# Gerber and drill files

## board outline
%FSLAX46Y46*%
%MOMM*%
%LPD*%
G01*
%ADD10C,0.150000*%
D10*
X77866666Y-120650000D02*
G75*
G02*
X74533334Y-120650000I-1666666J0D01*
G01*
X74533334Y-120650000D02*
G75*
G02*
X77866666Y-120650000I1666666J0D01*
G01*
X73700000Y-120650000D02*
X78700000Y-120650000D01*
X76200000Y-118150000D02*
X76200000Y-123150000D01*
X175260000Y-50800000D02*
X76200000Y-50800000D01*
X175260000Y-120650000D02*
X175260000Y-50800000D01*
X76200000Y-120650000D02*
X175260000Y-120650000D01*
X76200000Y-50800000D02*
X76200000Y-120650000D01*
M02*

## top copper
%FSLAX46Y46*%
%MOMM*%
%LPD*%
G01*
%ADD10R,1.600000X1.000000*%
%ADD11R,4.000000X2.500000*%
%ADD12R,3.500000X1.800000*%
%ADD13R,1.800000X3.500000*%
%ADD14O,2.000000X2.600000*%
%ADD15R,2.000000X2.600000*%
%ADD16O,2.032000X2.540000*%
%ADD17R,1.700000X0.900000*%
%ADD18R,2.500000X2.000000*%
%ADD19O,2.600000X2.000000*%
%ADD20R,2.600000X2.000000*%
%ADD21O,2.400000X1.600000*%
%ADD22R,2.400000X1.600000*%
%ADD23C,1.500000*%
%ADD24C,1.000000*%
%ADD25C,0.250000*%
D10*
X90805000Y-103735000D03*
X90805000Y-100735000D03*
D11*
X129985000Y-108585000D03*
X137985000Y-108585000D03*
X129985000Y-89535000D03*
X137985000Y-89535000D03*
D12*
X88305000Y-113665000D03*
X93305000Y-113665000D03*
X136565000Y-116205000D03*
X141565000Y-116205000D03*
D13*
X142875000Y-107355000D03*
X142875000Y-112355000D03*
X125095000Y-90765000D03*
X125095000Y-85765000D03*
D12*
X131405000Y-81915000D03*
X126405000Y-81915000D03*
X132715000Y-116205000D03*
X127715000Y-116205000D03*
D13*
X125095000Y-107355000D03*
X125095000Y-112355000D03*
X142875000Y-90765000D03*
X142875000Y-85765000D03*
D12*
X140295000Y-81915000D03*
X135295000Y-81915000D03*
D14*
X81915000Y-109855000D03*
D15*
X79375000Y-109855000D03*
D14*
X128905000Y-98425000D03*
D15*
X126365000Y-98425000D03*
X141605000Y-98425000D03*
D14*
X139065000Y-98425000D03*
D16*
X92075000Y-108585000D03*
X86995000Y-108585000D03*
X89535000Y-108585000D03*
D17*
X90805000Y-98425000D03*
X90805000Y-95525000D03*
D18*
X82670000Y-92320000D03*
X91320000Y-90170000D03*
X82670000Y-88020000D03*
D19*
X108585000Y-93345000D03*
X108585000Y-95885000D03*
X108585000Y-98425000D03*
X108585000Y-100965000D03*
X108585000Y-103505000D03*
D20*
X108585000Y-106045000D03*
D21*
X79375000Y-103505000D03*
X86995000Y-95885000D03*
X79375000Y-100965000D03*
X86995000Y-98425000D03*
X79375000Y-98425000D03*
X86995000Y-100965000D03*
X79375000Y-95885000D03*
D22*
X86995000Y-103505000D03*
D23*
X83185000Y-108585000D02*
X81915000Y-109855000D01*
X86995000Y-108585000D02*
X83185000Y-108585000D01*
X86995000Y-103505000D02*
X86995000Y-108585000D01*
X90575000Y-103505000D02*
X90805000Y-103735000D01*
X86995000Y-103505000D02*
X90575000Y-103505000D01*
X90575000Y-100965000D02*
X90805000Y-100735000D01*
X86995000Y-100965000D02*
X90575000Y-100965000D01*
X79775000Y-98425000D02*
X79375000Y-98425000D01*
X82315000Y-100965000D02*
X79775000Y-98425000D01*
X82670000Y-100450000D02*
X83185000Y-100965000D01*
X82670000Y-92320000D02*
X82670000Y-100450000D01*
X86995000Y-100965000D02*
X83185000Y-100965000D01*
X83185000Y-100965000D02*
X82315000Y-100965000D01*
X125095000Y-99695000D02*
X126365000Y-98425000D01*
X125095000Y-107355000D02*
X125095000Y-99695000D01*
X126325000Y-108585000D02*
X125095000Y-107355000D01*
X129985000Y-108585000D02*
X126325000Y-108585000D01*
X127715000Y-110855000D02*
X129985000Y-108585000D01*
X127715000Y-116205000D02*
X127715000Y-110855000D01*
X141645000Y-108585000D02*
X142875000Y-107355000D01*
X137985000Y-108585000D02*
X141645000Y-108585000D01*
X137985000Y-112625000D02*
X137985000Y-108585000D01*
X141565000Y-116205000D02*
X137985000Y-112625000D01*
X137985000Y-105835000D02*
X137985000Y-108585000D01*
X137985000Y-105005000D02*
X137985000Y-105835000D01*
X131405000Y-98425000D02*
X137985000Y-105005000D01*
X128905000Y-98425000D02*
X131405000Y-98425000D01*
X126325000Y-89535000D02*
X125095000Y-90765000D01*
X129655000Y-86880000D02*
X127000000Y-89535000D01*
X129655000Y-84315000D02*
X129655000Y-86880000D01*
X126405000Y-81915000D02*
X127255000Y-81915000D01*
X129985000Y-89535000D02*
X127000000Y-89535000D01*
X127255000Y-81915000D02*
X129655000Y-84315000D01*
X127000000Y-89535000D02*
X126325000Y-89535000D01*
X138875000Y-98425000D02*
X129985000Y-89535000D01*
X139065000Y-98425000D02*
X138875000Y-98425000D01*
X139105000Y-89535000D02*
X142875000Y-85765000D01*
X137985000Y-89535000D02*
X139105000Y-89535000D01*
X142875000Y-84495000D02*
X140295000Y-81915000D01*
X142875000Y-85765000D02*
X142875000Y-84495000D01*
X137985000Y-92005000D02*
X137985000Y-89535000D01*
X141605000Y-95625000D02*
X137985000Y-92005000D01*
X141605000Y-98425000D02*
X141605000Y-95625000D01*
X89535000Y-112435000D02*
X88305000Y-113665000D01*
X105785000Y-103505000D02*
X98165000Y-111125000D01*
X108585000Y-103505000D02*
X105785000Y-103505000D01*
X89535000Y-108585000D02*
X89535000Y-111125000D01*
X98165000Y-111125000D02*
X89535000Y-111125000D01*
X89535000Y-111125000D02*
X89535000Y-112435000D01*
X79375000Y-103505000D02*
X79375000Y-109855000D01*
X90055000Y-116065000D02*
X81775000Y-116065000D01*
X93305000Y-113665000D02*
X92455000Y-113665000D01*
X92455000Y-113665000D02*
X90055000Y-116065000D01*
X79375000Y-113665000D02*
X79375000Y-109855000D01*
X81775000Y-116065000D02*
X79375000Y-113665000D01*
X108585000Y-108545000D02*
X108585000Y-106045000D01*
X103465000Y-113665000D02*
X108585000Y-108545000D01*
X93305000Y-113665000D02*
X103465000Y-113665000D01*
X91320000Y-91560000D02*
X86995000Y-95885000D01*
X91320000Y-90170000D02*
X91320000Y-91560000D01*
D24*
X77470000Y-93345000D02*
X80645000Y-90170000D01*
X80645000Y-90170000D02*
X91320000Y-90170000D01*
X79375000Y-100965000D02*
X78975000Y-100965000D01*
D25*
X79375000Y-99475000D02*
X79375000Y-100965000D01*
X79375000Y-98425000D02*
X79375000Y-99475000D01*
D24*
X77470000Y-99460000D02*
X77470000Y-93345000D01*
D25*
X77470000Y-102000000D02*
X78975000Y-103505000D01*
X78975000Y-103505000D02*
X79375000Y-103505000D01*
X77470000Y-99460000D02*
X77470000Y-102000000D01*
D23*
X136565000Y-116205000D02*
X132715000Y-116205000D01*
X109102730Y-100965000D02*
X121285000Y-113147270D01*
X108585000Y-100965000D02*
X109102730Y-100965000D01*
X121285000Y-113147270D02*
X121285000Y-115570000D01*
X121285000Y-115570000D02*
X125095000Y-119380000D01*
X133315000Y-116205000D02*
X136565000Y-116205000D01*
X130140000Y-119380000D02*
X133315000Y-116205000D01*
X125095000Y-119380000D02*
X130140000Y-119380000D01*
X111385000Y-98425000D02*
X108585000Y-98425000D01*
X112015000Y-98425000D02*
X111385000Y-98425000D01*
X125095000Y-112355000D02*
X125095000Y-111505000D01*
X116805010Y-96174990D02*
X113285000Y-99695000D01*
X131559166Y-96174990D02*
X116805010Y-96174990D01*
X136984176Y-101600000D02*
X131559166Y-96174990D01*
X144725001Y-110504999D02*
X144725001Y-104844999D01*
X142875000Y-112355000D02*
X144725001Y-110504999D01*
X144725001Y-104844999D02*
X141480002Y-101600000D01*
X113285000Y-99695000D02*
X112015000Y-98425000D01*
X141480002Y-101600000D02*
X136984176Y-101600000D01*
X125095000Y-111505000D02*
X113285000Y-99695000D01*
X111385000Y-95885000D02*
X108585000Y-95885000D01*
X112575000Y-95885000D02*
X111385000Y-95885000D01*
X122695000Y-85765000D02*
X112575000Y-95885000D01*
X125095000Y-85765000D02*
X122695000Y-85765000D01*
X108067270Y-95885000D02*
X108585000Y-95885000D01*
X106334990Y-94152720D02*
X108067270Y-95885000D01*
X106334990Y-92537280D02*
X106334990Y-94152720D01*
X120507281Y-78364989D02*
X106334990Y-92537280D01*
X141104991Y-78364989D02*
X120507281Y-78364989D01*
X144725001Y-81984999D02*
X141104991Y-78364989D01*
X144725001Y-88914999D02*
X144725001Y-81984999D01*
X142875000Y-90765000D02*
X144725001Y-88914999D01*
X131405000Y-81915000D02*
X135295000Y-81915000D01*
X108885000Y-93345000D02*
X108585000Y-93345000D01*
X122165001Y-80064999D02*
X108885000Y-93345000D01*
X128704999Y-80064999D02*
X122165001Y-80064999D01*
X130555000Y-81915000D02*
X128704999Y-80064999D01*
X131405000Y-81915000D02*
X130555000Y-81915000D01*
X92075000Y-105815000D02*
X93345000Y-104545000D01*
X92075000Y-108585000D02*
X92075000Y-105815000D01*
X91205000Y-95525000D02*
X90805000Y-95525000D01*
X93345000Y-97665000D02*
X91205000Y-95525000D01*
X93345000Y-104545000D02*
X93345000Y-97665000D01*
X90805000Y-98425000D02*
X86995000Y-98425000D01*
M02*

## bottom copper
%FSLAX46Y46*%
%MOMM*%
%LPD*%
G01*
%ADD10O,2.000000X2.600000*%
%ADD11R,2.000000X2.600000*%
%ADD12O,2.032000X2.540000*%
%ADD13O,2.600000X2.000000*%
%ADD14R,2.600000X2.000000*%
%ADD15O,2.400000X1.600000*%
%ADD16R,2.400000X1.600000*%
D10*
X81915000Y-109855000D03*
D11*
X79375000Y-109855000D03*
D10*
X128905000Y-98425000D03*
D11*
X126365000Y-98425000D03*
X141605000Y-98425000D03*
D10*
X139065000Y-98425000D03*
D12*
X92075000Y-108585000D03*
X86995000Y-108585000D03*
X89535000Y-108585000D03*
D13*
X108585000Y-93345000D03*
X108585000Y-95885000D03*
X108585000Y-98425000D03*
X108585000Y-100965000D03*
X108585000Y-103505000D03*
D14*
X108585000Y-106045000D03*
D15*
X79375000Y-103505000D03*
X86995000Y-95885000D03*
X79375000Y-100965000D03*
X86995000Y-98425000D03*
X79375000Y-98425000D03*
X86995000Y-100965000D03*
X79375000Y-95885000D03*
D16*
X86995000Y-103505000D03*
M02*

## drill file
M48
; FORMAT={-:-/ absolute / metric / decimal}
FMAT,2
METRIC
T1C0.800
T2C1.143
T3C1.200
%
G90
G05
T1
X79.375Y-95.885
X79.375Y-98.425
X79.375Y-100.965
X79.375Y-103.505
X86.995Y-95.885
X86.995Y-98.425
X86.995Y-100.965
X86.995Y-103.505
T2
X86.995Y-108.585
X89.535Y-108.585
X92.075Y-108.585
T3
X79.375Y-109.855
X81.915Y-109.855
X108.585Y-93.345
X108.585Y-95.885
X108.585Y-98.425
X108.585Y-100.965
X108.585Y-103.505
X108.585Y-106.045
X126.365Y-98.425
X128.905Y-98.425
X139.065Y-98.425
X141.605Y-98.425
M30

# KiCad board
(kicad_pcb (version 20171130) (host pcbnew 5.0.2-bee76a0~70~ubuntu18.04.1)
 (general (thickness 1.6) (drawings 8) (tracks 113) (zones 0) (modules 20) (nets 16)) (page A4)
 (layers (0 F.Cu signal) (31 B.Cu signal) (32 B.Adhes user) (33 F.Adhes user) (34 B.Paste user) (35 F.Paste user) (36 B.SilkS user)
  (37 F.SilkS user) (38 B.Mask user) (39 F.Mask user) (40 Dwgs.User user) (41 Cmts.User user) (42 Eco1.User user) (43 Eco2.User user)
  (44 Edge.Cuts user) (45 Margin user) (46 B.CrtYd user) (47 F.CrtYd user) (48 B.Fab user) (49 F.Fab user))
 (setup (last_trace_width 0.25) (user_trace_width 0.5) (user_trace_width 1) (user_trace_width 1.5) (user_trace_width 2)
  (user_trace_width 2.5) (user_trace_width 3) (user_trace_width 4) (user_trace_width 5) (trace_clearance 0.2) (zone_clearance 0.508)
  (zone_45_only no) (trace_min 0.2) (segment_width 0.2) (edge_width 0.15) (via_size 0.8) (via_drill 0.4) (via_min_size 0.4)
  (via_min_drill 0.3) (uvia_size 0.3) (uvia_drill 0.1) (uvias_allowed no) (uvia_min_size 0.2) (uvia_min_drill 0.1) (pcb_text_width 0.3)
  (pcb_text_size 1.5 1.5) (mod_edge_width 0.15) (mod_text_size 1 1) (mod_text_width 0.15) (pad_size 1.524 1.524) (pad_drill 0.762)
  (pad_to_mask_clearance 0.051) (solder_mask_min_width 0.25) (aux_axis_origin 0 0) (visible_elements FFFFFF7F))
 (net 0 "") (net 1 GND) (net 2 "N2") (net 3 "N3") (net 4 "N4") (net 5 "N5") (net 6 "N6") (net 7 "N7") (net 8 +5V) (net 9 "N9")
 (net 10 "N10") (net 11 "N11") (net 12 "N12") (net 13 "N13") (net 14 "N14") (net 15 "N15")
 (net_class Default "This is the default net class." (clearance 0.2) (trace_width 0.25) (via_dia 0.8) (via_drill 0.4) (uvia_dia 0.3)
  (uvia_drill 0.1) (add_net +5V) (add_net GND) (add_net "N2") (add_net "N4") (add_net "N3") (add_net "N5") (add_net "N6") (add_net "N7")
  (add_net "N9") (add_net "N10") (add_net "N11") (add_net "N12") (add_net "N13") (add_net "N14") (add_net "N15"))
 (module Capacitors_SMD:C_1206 (layer F.Cu) (at 90.805 102.235 270)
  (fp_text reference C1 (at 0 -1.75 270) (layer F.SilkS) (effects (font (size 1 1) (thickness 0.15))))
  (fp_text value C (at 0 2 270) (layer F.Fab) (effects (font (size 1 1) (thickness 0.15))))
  (pad 2 smd rect (at 1.5 0 270) (size 1 1.6) (layers F.Cu F.Paste F.Mask) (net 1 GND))
  (pad 1 smd rect (at -1.5 0 270) (size 1 1.6) (layers F.Cu F.Paste F.Mask) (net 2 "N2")))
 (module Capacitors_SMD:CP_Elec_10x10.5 (layer F.Cu) (at 133.985 108.585 180)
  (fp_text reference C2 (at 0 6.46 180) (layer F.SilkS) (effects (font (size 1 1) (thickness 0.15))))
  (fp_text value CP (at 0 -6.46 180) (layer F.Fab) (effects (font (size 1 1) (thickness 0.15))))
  (pad 2 smd rect (at 4 0) (size 4 2.5) (layers F.Cu F.Paste F.Mask) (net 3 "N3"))
  (pad 1 smd rect (at -4 0) (size 4 2.5) (layers F.Cu F.Paste F.Mask) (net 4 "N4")))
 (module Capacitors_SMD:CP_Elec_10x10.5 (layer F.Cu) (at 133.985 89.535)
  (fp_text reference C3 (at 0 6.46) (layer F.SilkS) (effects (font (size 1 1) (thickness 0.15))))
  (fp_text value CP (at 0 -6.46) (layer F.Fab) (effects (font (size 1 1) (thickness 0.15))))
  (pad 1 smd rect (at -4 0 180) (size 4 2.5) (layers F.Cu F.Paste F.Mask) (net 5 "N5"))
  (pad 2 smd rect (at 4 0 180) (size 4 2.5) (layers F.Cu F.Paste F.Mask) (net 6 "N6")))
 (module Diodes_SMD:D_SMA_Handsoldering (layer F.Cu) (at 90.805 113.665 180)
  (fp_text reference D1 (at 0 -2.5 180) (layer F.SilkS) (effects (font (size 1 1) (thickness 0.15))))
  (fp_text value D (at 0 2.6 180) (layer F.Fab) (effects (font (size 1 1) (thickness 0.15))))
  (pad 2 smd rect (at 2.5 0 180) (size 3.5 1.8) (layers F.Cu F.Paste F.Mask) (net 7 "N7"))
  (pad 1 smd rect (at -2.5 0 180) (size 3.5 1.8) (layers F.Cu F.Paste F.Mask) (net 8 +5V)))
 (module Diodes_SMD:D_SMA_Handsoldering (layer F.Cu) (at 139.065 116.205 180)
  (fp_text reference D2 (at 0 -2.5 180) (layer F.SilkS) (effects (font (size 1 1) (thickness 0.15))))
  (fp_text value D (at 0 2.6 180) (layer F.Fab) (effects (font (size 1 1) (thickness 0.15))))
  (pad 2 smd rect (at 2.5 0 180) (size 3.5 1.8) (layers F.Cu F.Paste F.Mask) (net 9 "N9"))
  (pad 1 smd rect (at -2.5 0 180) (size 3.5 1.8) (layers F.Cu F.Paste F.Mask) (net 4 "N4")))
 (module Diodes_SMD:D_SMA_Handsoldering (layer F.Cu) (at 142.875 109.855 270)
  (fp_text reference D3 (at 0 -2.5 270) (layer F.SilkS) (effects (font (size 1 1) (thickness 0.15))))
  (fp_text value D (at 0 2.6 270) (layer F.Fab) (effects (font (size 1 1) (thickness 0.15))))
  (pad 1 smd rect (at -2.5 0 270) (size 3.5 1.8) (layers F.Cu F.Paste F.Mask) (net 4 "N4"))
  (pad 2 smd rect (at 2.5 0 270) (size 3.5 1.8) (layers F.Cu F.Paste F.Mask) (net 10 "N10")))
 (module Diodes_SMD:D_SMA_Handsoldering (layer F.Cu) (at 125.095 88.265 90)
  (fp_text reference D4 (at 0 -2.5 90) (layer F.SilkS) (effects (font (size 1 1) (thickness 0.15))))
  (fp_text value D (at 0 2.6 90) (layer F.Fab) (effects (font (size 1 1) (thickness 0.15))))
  (pad 1 smd rect (at -2.5 0 90) (size 3.5 1.8) (layers F.Cu F.Paste F.Mask) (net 5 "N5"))
  (pad 2 smd rect (at 2.5 0 90) (size 3.5 1.8) (layers F.Cu F.Paste F.Mask) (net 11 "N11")))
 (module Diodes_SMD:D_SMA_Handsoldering (layer F.Cu) (at 128.905 81.915)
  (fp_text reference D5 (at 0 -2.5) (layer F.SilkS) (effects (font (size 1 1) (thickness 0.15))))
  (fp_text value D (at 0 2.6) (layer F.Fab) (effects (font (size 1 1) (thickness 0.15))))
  (pad 2 smd rect (at 2.5 0) (size 3.5 1.8) (layers F.Cu F.Paste F.Mask) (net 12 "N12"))
  (pad 1 smd rect (at -2.5 0) (size 3.5 1.8) (layers F.Cu F.Paste F.Mask) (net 5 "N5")))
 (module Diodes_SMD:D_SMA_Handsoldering (layer F.Cu) (at 130.215 116.205 180)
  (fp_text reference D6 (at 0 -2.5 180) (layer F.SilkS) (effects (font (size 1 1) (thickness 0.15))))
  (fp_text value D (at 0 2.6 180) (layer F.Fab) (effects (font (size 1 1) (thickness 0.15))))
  (pad 1 smd rect (at -2.5 0 180) (size 3.5 1.8) (layers F.Cu F.Paste F.Mask) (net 9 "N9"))
  (pad 2 smd rect (at 2.5 0 180) (size 3.5 1.8) (layers F.Cu F.Paste F.Mask) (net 3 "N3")))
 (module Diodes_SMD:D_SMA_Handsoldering (layer F.Cu) (at 125.095 109.855 90)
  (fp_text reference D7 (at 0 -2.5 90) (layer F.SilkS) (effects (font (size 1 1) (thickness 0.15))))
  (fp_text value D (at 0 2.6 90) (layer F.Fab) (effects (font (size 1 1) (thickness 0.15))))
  (pad 2 smd rect (at 2.5 0 90) (size 3.5 1.8) (layers F.Cu F.Paste F.Mask) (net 3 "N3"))
  (pad 1 smd rect (at -2.5 0 90) (size 3.5 1.8) (layers F.Cu F.Paste F.Mask) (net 10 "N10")))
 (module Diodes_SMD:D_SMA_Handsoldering (layer F.Cu) (at 142.875 88.265 90)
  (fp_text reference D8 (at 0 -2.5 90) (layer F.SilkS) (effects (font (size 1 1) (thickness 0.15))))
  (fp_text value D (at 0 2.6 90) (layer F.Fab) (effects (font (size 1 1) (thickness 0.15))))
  (pad 1 smd rect (at -2.5 0 90) (size 3.5 1.8) (layers F.Cu F.Paste F.Mask) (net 11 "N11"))
  (pad 2 smd rect (at 2.5 0 90) (size 3.5 1.8) (layers F.Cu F.Paste F.Mask) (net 6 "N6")))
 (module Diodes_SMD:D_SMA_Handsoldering (layer F.Cu) (at 137.795 81.915)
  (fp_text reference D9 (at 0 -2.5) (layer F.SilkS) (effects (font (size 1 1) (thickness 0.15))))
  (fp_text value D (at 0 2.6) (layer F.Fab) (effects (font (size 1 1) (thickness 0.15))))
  (pad 2 smd rect (at 2.5 0) (size 3.5 1.8) (layers F.Cu F.Paste F.Mask) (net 6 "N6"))
  (pad 1 smd rect (at -2.5 0) (size 3.5 1.8) (layers F.Cu F.Paste F.Mask) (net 12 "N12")))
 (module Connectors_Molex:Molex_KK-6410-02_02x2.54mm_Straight (layer F.Cu) (at 79.375 109.855)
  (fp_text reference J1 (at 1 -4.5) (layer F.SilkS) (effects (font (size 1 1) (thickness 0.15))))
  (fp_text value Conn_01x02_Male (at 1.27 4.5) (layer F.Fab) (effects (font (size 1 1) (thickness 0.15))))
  (pad 2 thru_hole oval (at 2.54 0) (size 2 2.6) (drill 1.2) (layers *.Cu *.Mask) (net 1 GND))
  (pad 1 thru_hole rect (at 0 0) (size 2 2.6) (drill 1.2) (layers *.Cu *.Mask) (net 8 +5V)))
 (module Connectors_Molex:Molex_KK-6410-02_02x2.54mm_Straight (layer F.Cu) (at 126.365 98.425)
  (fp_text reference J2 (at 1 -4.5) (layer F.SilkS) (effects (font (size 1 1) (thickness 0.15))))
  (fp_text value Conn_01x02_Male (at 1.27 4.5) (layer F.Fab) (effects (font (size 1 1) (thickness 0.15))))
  (pad 2 thru_hole oval (at 2.54 0) (size 2 2.6) (drill 1.2) (layers *.Cu *.Mask) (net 4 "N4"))
  (pad 1 thru_hole rect (at 0 0) (size 2 2.6) (drill 1.2) (layers *.Cu *.Mask) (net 3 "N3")))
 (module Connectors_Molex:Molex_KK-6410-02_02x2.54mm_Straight (layer F.Cu) (at 141.605 98.425 180)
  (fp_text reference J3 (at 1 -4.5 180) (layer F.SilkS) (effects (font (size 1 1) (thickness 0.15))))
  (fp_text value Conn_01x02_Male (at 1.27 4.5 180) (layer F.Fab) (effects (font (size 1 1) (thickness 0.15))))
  (pad 1 thru_hole rect (at 0 0 180) (size 2 2.6) (drill 1.2) (layers *.Cu *.Mask) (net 6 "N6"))
  (pad 2 thru_hole oval (at 2.54 0 180) (size 2 2.6) (drill 1.2) (layers *.Cu *.Mask) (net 5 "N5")))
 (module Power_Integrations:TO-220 (layer F.Cu) (at 89.535 108.585 180)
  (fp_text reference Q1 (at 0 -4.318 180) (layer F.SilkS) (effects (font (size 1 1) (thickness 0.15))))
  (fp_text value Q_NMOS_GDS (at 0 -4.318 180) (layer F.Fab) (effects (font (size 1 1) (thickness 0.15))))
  (pad 1 thru_hole oval (at -2.54 0 180) (size 2.032 2.54) (drill 1.143) (layers *.Cu *.Mask) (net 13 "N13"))
  (pad 3 thru_hole oval (at 2.54 0 180) (size 2.032 2.54) (drill 1.143) (layers *.Cu *.Mask) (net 1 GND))
  (pad 2 thru_hole oval (at 0 0 180) (size 2.032 2.54) (drill 1.143) (layers *.Cu *.Mask) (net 7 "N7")))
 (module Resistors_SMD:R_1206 (layer F.Cu) (at 90.805 96.975 270)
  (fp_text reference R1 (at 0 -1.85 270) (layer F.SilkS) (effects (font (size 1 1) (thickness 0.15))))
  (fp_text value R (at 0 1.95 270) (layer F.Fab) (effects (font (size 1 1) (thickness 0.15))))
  (pad 2 smd rect (at 1.45 0 270) (size 0.9 1.7) (layers F.Cu F.Paste F.Mask) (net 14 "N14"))
  (pad 1 smd rect (at -1.45 0 270) (size 0.9 1.7) (layers F.Cu F.Paste F.Mask) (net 13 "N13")))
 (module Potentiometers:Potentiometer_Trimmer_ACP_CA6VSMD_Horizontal (layer F.Cu) (at 86.995 90.17)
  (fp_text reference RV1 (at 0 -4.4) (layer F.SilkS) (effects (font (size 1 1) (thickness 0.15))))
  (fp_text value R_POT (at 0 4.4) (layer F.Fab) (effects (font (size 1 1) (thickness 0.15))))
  (pad 1 smd rect (at -4.325 2.15) (size 2.5 2) (layers F.Cu F.Mask) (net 2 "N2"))
  (pad 2 smd rect (at 4.325 0) (size 2.5 2) (layers F.Cu F.Mask) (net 8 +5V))
  (pad 3 smd rect (at -4.325 -2.15) (size 2.5 2) (layers F.Cu F.Mask) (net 8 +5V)))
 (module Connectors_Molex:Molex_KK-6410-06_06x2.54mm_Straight (layer F.Cu) (at 108.585 106.045 90)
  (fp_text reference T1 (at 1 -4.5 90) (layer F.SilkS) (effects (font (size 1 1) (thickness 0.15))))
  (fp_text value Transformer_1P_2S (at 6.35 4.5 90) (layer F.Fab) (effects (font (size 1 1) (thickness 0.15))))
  (pad 6 thru_hole oval (at 12.7 0 90) (size 2 2.6) (drill 1.2) (layers *.Cu *.Mask) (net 12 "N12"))
  (pad 5 thru_hole oval (at 10.16 0 90) (size 2 2.6) (drill 1.2) (layers *.Cu *.Mask) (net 11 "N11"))
  (pad 4 thru_hole oval (at 7.62 0 90) (size 2 2.6) (drill 1.2) (layers *.Cu *.Mask) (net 10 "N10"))
  (pad 3 thru_hole oval (at 5.08 0 90) (size 2 2.6) (drill 1.2) (layers *.Cu *.Mask) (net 9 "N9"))
  (pad 2 thru_hole oval (at 2.54 0 90) (size 2 2.6) (drill 1.2) (layers *.Cu *.Mask) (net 7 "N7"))
  (pad 1 thru_hole rect (at 0 0 90) (size 2 2.6) (drill 1.2) (layers *.Cu *.Mask) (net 8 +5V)))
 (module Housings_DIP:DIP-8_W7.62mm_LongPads (layer F.Cu) (at 86.995 103.505 180)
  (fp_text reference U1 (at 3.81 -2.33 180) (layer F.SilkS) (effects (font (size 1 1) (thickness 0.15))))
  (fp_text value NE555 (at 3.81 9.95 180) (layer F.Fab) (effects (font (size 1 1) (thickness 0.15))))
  (pad 8 thru_hole oval (at 7.62 0 180) (size 2.4 1.6) (drill 0.8) (layers *.Cu *.Mask) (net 8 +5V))
  (pad 4 thru_hole oval (at 0 7.62 180) (size 2.4 1.6) (drill 0.8) (layers *.Cu *.Mask) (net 8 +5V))
  (pad 7 thru_hole oval (at 7.62 2.54 180) (size 2.4 1.6) (drill 0.8) (layers *.Cu *.Mask) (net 2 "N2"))
  (pad 3 thru_hole oval (at 0 5.08 180) (size 2.4 1.6) (drill 0.8) (layers *.Cu *.Mask) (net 14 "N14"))
  (pad 6 thru_hole oval (at 7.62 5.08 180) (size 2.4 1.6) (drill 0.8) (layers *.Cu *.Mask) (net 2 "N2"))
  (pad 2 thru_hole oval (at 0 2.54 180) (size 2.4 1.6) (drill 0.8) (layers *.Cu *.Mask) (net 2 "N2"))
  (pad 5 thru_hole oval (at 7.62 7.62 180) (size 2.4 1.6) (drill 0.8) (layers *.Cu *.Mask) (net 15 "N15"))
  (pad 1 thru_hole rect (at 0 0 180) (size 2.4 1.6) (drill 0.8) (layers *.Cu *.Mask) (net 1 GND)))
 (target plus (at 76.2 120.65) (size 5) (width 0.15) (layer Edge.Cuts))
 (gr_line (start 175.26 50.8) (end 76.2 50.8) (layer Edge.Cuts) (width 0.15))
 (gr_line (start 175.26 120.65) (end 175.26 50.8) (layer Edge.Cuts) (width 0.15))
 (gr_line (start 76.2 120.65) (end 175.26 120.65) (layer Edge.Cuts) (width 0.15))
 (gr_line (start 76.2 50.8) (end 76.2 120.65) (layer Edge.Cuts) (width 0.15))
 (segment (start 83.185 108.585) (end 81.915 109.855) (width 1.5) (layer F.Cu) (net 1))
 (segment (start 86.995 108.585) (end 83.185 108.585) (width 1.5) (layer F.Cu) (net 1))
 (segment (start 86.995 103.505) (end 86.995 108.585) (width 1.5) (layer F.Cu) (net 1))
 (segment (start 90.575 103.505) (end 90.805 103.735) (width 1.5) (layer F.Cu) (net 1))
 (segment (start 86.995 103.505) (end 90.575 103.505) (width 1.5) (layer F.Cu) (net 1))
 (segment (start 90.575 100.965) (end 90.805 100.735) (width 1.5) (layer F.Cu) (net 2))
 (segment (start 86.995 100.965) (end 90.575 100.965) (width 1.5) (layer F.Cu) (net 2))
 (segment (start 79.775 98.425) (end 79.375 98.425) (width 1.5) (layer F.Cu) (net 2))
 (segment (start 82.315 100.965) (end 79.775 98.425) (width 1.5) (layer F.Cu) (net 2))
 (segment (start 82.67 100.45) (end 83.185 100.965) (width 1.5) (layer F.Cu) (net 2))
 (segment (start 82.67 92.32) (end 82.67 100.45) (width 1.5) (layer F.Cu) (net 2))
 (segment (start 86.995 100.965) (end 83.185 100.965) (width 1.5) (layer F.Cu) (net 2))
 (segment (start 83.185 100.965) (end 82.315 100.965) (width 1.5) (layer F.Cu) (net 2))
 (segment (start 125.095 99.695) (end 126.365 98.425) (width 1.5) (layer F.Cu) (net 3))
 (segment (start 125.095 107.355) (end 125.095 99.695) (width 1.5) (layer F.Cu) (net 3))
 (segment (start 126.325 108.585) (end 125.095 107.355) (width 1.5) (layer F.Cu) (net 3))
 (segment (start 129.985 108.585) (end 126.325 108.585) (width 1.5) (layer F.Cu) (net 3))
 (segment (start 127.715 110.855) (end 129.985 108.585) (width 1.5) (layer F.Cu) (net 3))
 (segment (start 127.715 116.205) (end 127.715 110.855) (width 1.5) (layer F.Cu) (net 3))
 (segment (start 141.645 108.585) (end 142.875 107.355) (width 1.5) (layer F.Cu) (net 4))
 (segment (start 137.985 108.585) (end 141.645 108.585) (width 1.5) (layer F.Cu) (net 4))
 (segment (start 137.985 112.625) (end 137.985 108.585) (width 1.5) (layer F.Cu) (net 4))
 (segment (start 141.565 116.205) (end 137.985 112.625) (width 1.5) (layer F.Cu) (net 4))
 (segment (start 137.985 105.835) (end 137.985 108.585) (width 1.5) (layer F.Cu) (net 4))
 (segment (start 137.985 105.005) (end 137.985 105.835) (width 1.5) (layer F.Cu) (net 4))
 (segment (start 131.405 98.425) (end 137.985 105.005) (width 1.5) (layer F.Cu) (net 4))
 (segment (start 128.905 98.425) (end 131.405 98.425) (width 1.5) (layer F.Cu) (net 4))
 (segment (start 126.325 89.535) (end 125.095 90.765) (width 1.5) (layer F.Cu) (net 5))
 (segment (start 129.655 86.88) (end 127 89.535) (width 1.5) (layer F.Cu) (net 5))
 (segment (start 129.655 84.315) (end 129.655 86.88) (width 1.5) (layer F.Cu) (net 5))
 (segment (start 126.405 81.915) (end 127.255 81.915) (width 1.5) (layer F.Cu) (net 5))
 (segment (start 129.985 89.535) (end 127 89.535) (width 1.5) (layer F.Cu) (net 5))
 (segment (start 127.255 81.915) (end 129.655 84.315) (width 1.5) (layer F.Cu) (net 5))
 (segment (start 127 89.535) (end 126.325 89.535) (width 1.5) (layer F.Cu) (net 5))
 (segment (start 138.875 98.425) (end 129.985 89.535) (width 1.5) (layer F.Cu) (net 5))
 (segment (start 139.065 98.425) (end 138.875 98.425) (width 1.5) (layer F.Cu) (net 5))
 (segment (start 139.105 89.535) (end 142.875 85.765) (width 1.5) (layer F.Cu) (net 6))
 (segment (start 137.985 89.535) (end 139.105 89.535) (width 1.5) (layer F.Cu) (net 6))
 (segment (start 142.875 84.495) (end 140.295 81.915) (width 1.5) (layer F.Cu) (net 6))
 (segment (start 142.875 85.765) (end 142.875 84.495) (width 1.5) (layer F.Cu) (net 6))
 (segment (start 137.985 92.005) (end 137.985 89.535) (width 1.5) (layer F.Cu) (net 6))
 (segment (start 141.605 95.625) (end 137.985 92.005) (width 1.5) (layer F.Cu) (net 6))
 (segment (start 141.605 98.425) (end 141.605 95.625) (width 1.5) (layer F.Cu) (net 6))
 (segment (start 89.535 112.435) (end 88.305 113.665) (width 1.5) (layer F.Cu) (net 7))
 (segment (start 105.785 103.505) (end 98.165 111.125) (width 1.5) (layer F.Cu) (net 7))
 (segment (start 108.585 103.505) (end 105.785 103.505) (width 1.5) (layer F.Cu) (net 7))
 (segment (start 89.535 108.585) (end 89.535 111.125) (width 1.5) (layer F.Cu) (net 7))
 (segment (start 98.165 111.125) (end 89.535 111.125) (width 1.5) (layer F.Cu) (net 7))
 (segment (start 89.535 111.125) (end 89.535 112.435) (width 1.5) (layer F.Cu) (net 7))
 (segment (start 79.375 103.505) (end 79.375 109.855) (width 1.5) (layer F.Cu) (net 8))
 (segment (start 90.055 116.065) (end 81.775 116.065) (width 1.5) (layer F.Cu) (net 8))
 (segment (start 93.305 113.665) (end 92.455 113.665) (width 1.5) (layer F.Cu) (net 8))
 (segment (start 92.455 113.665) (end 90.055 116.065) (width 1.5) (layer F.Cu) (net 8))
 (segment (start 79.375 113.665) (end 79.375 109.855) (width 1.5) (layer F.Cu) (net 8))
 (segment (start 81.775 116.065) (end 79.375 113.665) (width 1.5) (layer F.Cu) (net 8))
 (segment (start 108.585 108.545) (end 108.585 106.045) (width 1.5) (layer F.Cu) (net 8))
 (segment (start 103.465 113.665) (end 108.585 108.545) (width 1.5) (layer F.Cu) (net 8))
 (segment (start 93.305 113.665) (end 103.465 113.665) (width 1.5) (layer F.Cu) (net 8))
 (segment (start 91.32 91.56) (end 86.995 95.885) (width 1.5) (layer F.Cu) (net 8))
 (segment (start 91.32 90.17) (end 91.32 91.56) (width 1.5) (layer F.Cu) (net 8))
 (segment (start 77.47 93.345) (end 80.645 90.17) (width 1) (layer F.Cu) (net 8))
 (segment (start 80.645 90.17) (end 91.32 90.17) (width 1) (layer F.Cu) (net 8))
 (segment (start 79.375 100.965) (end 78.975 100.965) (width 1) (layer F.Cu) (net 2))
 (segment (start 79.375 99.475) (end 79.375 100.965) (width 0.25) (layer F.Cu) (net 2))
 (segment (start 79.375 98.425) (end 79.375 99.475) (width 0.25) (layer F.Cu) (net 2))
 (segment (start 77.47 99.46) (end 77.47 93.345) (width 1) (layer F.Cu) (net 8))
 (segment (start 77.47 102) (end 78.975 103.505) (width 0.25) (layer F.Cu) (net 8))
 (segment (start 78.975 103.505) (end 79.375 103.505) (width 0.25) (layer F.Cu) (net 8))
 (segment (start 77.47 99.46) (end 77.47 102) (width 0.25) (layer F.Cu) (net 8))
 (segment (start 136.565 116.205) (end 132.715 116.205) (width 1.5) (layer F.Cu) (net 9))
 (segment (start 109.10273 100.965) (end 121.285 113.14727) (width 1.5) (layer F.Cu) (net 9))
 (segment (start 108.585 100.965) (end 109.10273 100.965) (width 1.5) (layer F.Cu) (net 9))
 (segment (start 121.285 113.14727) (end 121.285 115.57) (width 1.5) (layer F.Cu) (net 9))
 (segment (start 121.285 115.57) (end 125.095 119.38) (width 1.5) (layer F.Cu) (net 9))
 (segment (start 133.315 116.205) (end 136.565 116.205) (width 1.5) (layer F.Cu) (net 9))
 (segment (start 130.14 119.38) (end 133.315 116.205) (width 1.5) (layer F.Cu) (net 9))
 (segment (start 125.095 119.38) (end 130.14 119.38) (width 1.5) (layer F.Cu) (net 9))
 (segment (start 111.385 98.425) (end 108.585 98.425) (width 1.5) (layer F.Cu) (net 10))
 (segment (start 112.015 98.425) (end 111.385 98.425) (width 1.5) (layer F.Cu) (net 10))
 (segment (start 125.095 112.355) (end 125.095 111.505) (width 1.5) (layer F.Cu) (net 10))
 (segment (start 116.80501 96.17499) (end 113.285 99.695) (width 1.5) (layer F.Cu) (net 10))
 (segment (start 131.559166 96.17499) (end 116.80501 96.17499) (width 1.5) (layer F.Cu) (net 10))
 (segment (start 136.984176 101.6) (end 131.559166 96.17499) (width 1.5) (layer F.Cu) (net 10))
 (segment (start 144.725001 110.504999) (end 144.725001 104.844999) (width 1.5) (layer F.Cu) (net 10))
 (segment (start 142.875 112.355) (end 144.725001 110.504999) (width 1.5) (layer F.Cu) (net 10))
 (segment (start 144.725001 104.844999) (end 141.480002 101.6) (width 1.5) (layer F.Cu) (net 10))
 (segment (start 113.285 99.695) (end 112.015 98.425) (width 1.5) (layer F.Cu) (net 10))
 (segment (start 141.480002 101.6) (end 136.984176 101.6) (width 1.5) (layer F.Cu) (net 10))
 (segment (start 125.095 111.505) (end 113.285 99.695) (width 1.5) (layer F.Cu) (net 10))
 (segment (start 111.385 95.885) (end 108.585 95.885) (width 1.5) (layer F.Cu) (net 11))
 (segment (start 112.575 95.885) (end 111.385 95.885) (width 1.5) (layer F.Cu) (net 11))
 (segment (start 122.695 85.765) (end 112.575 95.885) (width 1.5) (layer F.Cu) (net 11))
 (segment (start 125.095 85.765) (end 122.695 85.765) (width 1.5) (layer F.Cu) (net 11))
 (segment (start 108.06727 95.885) (end 108.585 95.885) (width 1.5) (layer F.Cu) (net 11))
 (segment (start 106.33499 94.15272) (end 108.06727 95.885) (width 1.5) (layer F.Cu) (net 11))
 (segment (start 106.33499 92.53728) (end 106.33499 94.15272) (width 1.5) (layer F.Cu) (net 11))
 (segment (start 120.507281 78.364989) (end 106.33499 92.53728) (width 1.5) (layer F.Cu) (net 11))
 (segment (start 141.104991 78.364989) (end 120.507281 78.364989) (width 1.5) (layer F.Cu) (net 11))
 (segment (start 144.725001 81.984999) (end 141.104991 78.364989) (width 1.5) (layer F.Cu) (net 11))
 (segment (start 144.725001 88.914999) (end 144.725001 81.984999) (width 1.5) (layer F.Cu) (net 11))
 (segment (start 142.875 90.765) (end 144.725001 88.914999) (width 1.5) (layer F.Cu) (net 11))
 (segment (start 131.405 81.915) (end 135.295 81.915) (width 1.5) (layer F.Cu) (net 12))
 (segment (start 108.885 93.345) (end 108.585 93.345) (width 1.5) (layer F.Cu) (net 12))
 (segment (start 122.165001 80.064999) (end 108.885 93.345) (width 1.5) (layer F.Cu) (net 12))
 (segment (start 128.704999 80.064999) (end 122.165001 80.064999) (width 1.5) (layer F.Cu) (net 12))
 (segment (start 130.555 81.915) (end 128.704999 80.064999) (width 1.5) (layer F.Cu) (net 12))
 (segment (start 131.405 81.915) (end 130.555 81.915) (width 1.5) (layer F.Cu) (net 12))
 (segment (start 92.075 105.815) (end 93.345 104.545) (width 1.5) (layer F.Cu) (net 13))
 (segment (start 92.075 108.585) (end 92.075 105.815) (width 1.5) (layer F.Cu) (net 13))
 (segment (start 91.205 95.525) (end 90.805 95.525) (width 1.5) (layer F.Cu) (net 13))
 (segment (start 93.345 97.665) (end 91.205 95.525) (width 1.5) (layer F.Cu) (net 13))
 (segment (start 93.345 104.545) (end 93.345 97.665) (width 1.5) (layer F.Cu) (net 13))
 (segment (start 90.805 98.425) (end 86.995 98.425) (width 1.5) (layer F.Cu) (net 14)))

